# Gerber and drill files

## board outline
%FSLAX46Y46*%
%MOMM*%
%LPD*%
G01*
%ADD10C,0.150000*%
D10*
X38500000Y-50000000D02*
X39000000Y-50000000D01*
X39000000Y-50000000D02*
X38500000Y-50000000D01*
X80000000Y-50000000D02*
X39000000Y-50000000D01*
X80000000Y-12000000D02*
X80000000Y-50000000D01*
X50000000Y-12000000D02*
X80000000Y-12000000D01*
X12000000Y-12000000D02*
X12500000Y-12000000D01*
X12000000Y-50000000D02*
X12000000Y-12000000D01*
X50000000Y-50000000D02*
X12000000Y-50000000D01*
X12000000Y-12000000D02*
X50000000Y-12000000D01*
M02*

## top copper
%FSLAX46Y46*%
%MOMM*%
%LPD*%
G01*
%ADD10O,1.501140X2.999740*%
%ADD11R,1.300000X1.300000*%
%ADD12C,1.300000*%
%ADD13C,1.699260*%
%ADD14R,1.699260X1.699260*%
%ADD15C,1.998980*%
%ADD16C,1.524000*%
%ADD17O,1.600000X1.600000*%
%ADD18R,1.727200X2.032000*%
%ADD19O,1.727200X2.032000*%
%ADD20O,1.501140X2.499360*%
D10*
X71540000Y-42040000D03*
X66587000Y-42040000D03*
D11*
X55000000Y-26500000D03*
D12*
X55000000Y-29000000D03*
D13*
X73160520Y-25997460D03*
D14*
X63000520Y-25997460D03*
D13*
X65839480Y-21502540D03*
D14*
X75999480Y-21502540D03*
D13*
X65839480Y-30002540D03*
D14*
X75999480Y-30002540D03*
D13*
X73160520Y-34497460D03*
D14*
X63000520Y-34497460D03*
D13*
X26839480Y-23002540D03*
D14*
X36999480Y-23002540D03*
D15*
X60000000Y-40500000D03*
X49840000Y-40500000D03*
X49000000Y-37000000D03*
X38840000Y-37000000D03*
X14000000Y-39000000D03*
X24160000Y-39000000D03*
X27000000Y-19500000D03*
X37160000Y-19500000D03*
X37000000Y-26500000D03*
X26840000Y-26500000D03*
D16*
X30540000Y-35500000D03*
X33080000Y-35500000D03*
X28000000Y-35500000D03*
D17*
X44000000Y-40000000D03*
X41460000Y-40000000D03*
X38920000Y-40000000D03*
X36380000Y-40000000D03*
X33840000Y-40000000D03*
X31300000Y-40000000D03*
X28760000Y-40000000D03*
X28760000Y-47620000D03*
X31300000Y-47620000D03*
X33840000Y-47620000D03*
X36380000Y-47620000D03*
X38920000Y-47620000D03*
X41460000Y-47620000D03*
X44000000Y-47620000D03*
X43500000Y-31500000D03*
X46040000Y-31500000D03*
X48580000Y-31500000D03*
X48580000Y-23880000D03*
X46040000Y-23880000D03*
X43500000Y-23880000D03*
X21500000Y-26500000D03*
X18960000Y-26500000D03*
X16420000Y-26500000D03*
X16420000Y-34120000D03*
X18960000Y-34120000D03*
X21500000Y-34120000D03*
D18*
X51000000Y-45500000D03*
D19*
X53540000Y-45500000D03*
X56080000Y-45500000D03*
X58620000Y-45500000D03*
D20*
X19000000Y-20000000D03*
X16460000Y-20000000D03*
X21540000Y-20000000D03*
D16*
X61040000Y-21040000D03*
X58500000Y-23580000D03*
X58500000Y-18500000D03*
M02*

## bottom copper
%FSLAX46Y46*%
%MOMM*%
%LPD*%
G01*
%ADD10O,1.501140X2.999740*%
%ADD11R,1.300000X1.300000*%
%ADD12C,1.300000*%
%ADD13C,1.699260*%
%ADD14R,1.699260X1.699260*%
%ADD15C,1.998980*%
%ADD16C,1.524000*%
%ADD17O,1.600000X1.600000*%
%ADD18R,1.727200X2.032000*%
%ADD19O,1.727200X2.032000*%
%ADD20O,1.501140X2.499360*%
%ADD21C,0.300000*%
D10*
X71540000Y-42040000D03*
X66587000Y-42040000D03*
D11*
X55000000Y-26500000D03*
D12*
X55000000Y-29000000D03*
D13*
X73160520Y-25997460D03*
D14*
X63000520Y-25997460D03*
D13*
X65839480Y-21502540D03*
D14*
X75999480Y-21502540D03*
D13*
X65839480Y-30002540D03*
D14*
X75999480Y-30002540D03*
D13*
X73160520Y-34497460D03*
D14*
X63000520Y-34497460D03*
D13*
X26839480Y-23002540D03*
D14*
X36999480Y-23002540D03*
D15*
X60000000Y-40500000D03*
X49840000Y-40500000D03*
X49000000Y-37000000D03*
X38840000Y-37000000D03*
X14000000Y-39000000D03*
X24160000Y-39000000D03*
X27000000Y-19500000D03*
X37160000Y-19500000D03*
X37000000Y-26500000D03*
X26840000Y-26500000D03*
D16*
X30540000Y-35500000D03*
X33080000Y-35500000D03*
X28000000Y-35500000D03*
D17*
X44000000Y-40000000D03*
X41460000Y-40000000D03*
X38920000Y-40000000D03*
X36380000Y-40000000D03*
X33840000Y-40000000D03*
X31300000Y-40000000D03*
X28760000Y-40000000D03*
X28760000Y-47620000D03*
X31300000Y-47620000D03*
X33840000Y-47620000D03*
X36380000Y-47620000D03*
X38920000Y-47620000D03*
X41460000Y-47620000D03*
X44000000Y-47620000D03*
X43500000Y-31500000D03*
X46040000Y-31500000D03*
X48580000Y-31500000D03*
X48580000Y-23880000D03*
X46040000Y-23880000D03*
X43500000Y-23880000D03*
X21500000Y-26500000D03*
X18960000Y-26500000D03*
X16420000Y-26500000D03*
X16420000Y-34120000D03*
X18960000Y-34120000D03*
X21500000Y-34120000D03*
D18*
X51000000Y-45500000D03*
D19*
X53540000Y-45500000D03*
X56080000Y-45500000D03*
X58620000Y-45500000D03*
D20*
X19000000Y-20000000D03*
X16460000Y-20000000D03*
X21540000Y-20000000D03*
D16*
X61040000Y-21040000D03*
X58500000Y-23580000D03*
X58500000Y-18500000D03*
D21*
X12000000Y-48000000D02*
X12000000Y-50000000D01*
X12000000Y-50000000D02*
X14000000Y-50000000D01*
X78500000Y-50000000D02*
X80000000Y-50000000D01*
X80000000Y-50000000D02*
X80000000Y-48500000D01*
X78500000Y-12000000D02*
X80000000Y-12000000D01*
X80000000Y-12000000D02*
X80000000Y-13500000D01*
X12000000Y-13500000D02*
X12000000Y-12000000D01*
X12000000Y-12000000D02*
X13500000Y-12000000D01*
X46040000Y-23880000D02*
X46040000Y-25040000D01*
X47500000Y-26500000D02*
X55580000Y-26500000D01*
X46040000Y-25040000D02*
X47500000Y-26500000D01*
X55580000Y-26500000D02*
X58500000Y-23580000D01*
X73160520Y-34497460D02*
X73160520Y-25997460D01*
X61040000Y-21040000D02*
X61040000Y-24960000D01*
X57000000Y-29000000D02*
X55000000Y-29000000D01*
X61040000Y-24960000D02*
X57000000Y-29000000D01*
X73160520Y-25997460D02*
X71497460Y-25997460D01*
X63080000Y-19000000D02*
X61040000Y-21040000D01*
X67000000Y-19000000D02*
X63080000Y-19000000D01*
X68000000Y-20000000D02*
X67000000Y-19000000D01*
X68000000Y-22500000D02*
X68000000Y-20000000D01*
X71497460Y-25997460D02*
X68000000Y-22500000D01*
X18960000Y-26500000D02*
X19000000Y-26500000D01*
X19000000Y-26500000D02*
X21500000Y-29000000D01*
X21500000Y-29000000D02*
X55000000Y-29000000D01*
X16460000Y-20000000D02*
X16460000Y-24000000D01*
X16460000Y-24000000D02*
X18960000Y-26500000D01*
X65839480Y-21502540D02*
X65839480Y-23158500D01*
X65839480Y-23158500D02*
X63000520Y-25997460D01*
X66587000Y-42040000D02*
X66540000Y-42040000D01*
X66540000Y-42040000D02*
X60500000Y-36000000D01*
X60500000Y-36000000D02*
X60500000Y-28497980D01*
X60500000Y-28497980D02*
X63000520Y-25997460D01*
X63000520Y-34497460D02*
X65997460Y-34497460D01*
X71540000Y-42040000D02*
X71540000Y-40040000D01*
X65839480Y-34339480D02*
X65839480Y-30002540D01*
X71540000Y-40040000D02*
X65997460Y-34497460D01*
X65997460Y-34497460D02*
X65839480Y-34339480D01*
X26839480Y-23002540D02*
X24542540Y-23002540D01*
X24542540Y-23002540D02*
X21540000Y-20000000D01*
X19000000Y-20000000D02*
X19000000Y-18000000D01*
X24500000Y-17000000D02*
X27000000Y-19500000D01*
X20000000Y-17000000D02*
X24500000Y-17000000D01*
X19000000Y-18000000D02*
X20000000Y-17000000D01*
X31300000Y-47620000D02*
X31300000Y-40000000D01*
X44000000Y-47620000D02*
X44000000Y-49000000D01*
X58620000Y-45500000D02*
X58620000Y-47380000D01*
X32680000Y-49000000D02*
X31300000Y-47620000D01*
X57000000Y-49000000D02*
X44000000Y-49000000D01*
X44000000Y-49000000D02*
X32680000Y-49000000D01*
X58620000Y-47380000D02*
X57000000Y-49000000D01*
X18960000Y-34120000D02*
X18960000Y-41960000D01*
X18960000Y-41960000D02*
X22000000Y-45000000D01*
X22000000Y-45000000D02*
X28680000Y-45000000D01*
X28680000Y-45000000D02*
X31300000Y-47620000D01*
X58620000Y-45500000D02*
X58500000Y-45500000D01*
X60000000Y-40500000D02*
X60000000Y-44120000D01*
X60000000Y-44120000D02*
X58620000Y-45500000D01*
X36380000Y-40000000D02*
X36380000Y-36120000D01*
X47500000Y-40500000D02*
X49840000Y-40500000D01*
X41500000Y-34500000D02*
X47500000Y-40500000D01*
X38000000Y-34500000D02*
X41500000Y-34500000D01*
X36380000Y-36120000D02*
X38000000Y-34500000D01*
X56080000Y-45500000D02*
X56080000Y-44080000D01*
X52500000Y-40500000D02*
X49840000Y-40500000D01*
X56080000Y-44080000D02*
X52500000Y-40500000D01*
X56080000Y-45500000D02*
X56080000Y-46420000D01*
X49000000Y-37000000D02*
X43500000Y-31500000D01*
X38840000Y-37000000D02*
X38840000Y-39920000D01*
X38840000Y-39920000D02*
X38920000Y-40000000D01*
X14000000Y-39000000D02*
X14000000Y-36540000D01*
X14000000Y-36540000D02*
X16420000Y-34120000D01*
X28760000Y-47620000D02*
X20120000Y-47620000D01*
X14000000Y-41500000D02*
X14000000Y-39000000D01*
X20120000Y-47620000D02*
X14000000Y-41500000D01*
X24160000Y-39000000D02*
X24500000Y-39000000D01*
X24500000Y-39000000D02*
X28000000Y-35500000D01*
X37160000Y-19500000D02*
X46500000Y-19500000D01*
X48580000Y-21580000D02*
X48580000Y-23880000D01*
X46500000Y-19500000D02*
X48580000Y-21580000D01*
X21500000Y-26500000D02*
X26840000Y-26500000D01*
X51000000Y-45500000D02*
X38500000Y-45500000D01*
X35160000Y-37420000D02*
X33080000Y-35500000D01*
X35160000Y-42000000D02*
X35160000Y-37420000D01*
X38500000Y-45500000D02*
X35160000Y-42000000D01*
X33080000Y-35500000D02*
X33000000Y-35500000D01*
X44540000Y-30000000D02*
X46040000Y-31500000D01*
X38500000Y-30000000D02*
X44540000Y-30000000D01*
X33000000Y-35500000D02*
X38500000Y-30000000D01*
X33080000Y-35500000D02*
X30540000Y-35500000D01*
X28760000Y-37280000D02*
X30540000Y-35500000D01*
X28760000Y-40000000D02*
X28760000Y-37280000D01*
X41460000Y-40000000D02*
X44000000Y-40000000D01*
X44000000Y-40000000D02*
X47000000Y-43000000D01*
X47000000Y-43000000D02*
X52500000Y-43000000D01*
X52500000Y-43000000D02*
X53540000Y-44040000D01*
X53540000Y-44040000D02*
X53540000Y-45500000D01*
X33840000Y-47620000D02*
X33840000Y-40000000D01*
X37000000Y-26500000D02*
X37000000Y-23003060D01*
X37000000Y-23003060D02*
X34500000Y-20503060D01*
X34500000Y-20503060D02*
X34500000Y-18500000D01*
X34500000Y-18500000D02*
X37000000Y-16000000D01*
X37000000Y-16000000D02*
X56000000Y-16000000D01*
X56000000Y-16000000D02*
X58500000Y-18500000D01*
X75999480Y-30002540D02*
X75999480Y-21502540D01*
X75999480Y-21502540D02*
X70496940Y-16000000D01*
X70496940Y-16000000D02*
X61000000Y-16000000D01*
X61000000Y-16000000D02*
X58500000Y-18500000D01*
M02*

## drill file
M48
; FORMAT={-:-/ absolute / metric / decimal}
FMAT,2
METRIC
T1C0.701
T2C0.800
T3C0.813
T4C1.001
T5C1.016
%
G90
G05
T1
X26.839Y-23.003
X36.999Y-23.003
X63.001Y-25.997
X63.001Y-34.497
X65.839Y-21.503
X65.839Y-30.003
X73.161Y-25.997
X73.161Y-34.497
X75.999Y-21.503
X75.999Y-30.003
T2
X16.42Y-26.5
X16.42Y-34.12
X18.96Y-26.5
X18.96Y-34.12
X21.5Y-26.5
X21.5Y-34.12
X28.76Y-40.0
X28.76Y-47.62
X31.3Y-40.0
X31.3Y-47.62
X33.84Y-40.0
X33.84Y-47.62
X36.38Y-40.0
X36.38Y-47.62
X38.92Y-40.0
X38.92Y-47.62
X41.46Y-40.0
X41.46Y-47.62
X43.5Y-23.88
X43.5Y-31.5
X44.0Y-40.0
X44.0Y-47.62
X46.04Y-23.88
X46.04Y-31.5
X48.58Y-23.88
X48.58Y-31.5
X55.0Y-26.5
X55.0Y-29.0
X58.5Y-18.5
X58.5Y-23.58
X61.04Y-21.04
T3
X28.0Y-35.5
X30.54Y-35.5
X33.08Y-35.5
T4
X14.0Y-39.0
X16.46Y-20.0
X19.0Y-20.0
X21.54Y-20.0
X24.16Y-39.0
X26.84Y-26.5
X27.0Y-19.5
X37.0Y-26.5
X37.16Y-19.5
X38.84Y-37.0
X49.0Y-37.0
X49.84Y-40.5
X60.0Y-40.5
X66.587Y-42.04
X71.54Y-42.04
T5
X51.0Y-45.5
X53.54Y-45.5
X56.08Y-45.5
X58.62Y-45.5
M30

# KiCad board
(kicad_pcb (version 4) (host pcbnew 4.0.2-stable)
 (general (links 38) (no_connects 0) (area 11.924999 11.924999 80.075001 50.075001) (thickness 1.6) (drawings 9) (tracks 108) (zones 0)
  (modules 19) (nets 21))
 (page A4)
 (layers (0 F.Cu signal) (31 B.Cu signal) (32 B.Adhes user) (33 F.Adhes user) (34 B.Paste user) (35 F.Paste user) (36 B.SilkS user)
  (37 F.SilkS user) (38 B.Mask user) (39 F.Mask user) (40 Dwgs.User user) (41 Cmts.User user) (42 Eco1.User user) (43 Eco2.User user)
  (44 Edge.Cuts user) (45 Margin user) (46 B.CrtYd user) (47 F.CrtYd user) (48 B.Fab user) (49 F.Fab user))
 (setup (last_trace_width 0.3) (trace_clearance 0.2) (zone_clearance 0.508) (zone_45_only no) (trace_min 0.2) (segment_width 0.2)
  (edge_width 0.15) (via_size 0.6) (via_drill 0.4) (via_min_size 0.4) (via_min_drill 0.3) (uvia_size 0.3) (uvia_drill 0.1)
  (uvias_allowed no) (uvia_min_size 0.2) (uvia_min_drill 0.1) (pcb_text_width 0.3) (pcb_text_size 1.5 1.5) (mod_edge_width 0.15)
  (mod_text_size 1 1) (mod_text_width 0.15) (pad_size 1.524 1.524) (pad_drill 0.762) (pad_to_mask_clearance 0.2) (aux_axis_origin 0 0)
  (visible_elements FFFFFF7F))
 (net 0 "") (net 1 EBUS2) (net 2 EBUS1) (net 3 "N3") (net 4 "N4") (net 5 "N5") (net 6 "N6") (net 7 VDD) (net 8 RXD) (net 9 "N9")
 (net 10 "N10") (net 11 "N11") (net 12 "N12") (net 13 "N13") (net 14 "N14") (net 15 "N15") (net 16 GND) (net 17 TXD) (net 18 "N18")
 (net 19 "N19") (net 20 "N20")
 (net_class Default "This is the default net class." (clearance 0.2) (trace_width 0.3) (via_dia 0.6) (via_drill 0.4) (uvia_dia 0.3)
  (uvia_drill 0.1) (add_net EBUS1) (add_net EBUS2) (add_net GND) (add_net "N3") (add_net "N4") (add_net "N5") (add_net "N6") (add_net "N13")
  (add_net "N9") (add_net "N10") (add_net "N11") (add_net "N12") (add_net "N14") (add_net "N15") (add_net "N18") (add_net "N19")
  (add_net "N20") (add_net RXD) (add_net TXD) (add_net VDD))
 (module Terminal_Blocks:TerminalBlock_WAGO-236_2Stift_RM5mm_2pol (layer F.Cu) (at 69 39.5 180)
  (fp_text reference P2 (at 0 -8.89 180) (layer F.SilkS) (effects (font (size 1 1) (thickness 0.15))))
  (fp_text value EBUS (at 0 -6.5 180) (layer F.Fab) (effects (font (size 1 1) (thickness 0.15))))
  (pad 1 thru_hole oval (at -2.54 -2.54 270) (size 2.99974 1.50114) (drill 1.00076) (layers *.Cu *.Mask F.SilkS) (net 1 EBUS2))
  (pad 2 thru_hole oval (at 2.413 -2.54 270) (size 2.99974 1.50114) (drill 1.00076) (layers *.Cu *.Mask F.SilkS) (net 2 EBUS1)))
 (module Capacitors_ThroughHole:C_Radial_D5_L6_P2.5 (layer F.Cu) (at 55 26.5 270)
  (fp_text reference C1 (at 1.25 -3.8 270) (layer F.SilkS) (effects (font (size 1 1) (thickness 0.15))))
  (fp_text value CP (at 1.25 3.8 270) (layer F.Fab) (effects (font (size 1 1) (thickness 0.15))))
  (pad 1 thru_hole rect (at 0 0 270) (size 1.3 1.3) (drill 0.8) (layers *.Cu *.Mask F.SilkS) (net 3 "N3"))
  (pad 2 thru_hole circle (at 2.5 0 270) (size 1.3 1.3) (drill 0.8) (layers *.Cu *.Mask F.SilkS) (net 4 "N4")))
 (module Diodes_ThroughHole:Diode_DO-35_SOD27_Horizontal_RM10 (layer F.Cu) (at 63 26)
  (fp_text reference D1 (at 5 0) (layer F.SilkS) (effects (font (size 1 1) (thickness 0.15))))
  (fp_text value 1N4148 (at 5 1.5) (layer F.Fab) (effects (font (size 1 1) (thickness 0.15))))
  (pad 2 thru_hole circle (at 10.16052 -0.00254 180) (size 1.69926 1.69926) (drill 0.70104) (layers *.Cu *.Mask F.SilkS) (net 4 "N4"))
  (pad 1 thru_hole rect (at 0.00052 -0.00254 180) (size 1.69926 1.69926) (drill 0.70104) (layers *.Cu *.Mask F.SilkS) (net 2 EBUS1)))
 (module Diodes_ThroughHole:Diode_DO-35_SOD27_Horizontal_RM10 (layer F.Cu) (at 76 21.5 180)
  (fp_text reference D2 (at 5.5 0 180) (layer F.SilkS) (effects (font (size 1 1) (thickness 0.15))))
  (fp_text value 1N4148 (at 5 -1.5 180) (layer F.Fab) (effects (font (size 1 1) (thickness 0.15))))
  (pad 2 thru_hole circle (at 10.16052 -0.00254) (size 1.69926 1.69926) (drill 0.70104) (layers *.Cu *.Mask F.SilkS) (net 2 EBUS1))
  (pad 1 thru_hole rect (at 0.00052 -0.00254) (size 1.69926 1.69926) (drill 0.70104) (layers *.Cu *.Mask F.SilkS) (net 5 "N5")))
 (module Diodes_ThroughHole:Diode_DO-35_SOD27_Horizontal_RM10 (layer F.Cu) (at 76 30 180)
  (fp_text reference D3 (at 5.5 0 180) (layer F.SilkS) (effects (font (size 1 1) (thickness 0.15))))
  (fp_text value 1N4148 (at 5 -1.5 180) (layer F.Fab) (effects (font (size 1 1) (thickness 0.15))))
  (pad 2 thru_hole circle (at 10.16052 -0.00254) (size 1.69926 1.69926) (drill 0.70104) (layers *.Cu *.Mask F.SilkS) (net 1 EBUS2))
  (pad 1 thru_hole rect (at 0.00052 -0.00254) (size 1.69926 1.69926) (drill 0.70104) (layers *.Cu *.Mask F.SilkS) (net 5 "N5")))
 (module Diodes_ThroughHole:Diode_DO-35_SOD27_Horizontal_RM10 (layer F.Cu) (at 63 34.5)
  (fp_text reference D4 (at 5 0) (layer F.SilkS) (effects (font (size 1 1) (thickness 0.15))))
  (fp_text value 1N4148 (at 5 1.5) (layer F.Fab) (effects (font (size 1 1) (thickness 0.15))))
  (pad 2 thru_hole circle (at 10.16052 -0.00254 180) (size 1.69926 1.69926) (drill 0.70104) (layers *.Cu *.Mask F.SilkS) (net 4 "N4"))
  (pad 1 thru_hole rect (at 0.00052 -0.00254 180) (size 1.69926 1.69926) (drill 0.70104) (layers *.Cu *.Mask F.SilkS) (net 1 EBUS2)))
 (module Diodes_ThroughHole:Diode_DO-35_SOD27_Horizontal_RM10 (layer F.Cu) (at 37 23 180)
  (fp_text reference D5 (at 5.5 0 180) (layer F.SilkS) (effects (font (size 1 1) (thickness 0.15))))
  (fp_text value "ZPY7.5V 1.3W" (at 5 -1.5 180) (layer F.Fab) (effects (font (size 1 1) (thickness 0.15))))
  (pad 2 thru_hole circle (at 10.16052 -0.00254) (size 1.69926 1.69926) (drill 0.70104) (layers *.Cu *.Mask F.SilkS) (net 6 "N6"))
  (pad 1 thru_hole rect (at 0.00052 -0.00254) (size 1.69926 1.69926) (drill 0.70104) (layers *.Cu *.Mask F.SilkS) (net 5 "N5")))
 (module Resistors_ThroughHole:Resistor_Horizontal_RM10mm (layer F.Cu) (at 60 40.5 180)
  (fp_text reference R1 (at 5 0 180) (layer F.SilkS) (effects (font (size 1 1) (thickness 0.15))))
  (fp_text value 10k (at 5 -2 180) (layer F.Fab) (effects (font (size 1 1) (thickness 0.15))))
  (pad 1 thru_hole circle (at 0 0 180) (size 1.99898 1.99898) (drill 1.00076) (layers *.Cu *.SilkS *.Mask) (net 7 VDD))
  (pad 2 thru_hole circle (at 10.16 0 180) (size 1.99898 1.99898) (drill 1.00076) (layers *.Cu *.SilkS *.Mask) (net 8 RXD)))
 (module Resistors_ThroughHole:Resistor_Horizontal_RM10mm (layer F.Cu) (at 49 37 180)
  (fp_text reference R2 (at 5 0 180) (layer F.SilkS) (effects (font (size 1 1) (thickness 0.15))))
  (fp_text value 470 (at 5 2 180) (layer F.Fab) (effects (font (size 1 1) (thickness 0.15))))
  (pad 1 thru_hole circle (at 0 0 180) (size 1.99898 1.99898) (drill 1.00076) (layers *.Cu *.SilkS *.Mask) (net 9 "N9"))
  (pad 2 thru_hole circle (at 10.16 0 180) (size 1.99898 1.99898) (drill 1.00076) (layers *.Cu *.SilkS *.Mask) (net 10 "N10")))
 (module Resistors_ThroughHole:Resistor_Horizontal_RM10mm (layer F.Cu) (at 14 39)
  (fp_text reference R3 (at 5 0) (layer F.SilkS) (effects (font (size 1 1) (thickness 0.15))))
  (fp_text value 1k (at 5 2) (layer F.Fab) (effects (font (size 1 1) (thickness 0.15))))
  (pad 1 thru_hole circle (at 0 0) (size 1.99898 1.99898) (drill 1.00076) (layers *.Cu *.SilkS *.Mask) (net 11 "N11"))
  (pad 2 thru_hole circle (at 10.16 0) (size 1.99898 1.99898) (drill 1.00076) (layers *.Cu *.SilkS *.Mask) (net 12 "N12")))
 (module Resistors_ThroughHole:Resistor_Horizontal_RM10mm (layer F.Cu) (at 27 19.5)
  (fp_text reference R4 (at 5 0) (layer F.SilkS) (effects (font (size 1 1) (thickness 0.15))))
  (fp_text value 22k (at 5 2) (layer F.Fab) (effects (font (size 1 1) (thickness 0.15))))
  (pad 1 thru_hole circle (at 0 0) (size 1.99898 1.99898) (drill 1.00076) (layers *.Cu *.SilkS *.Mask) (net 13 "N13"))
  (pad 2 thru_hole circle (at 10.16 0) (size 1.99898 1.99898) (drill 1.00076) (layers *.Cu *.SilkS *.Mask) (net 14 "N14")))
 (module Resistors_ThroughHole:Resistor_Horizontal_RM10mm (layer F.Cu) (at 37 26.5 180)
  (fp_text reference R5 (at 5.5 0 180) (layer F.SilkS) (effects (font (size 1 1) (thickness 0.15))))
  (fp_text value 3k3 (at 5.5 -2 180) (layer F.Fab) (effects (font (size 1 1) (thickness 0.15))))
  (pad 1 thru_hole circle (at 0 0 180) (size 1.99898 1.99898) (drill 1.00076) (layers *.Cu *.SilkS *.Mask) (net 5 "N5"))
  (pad 2 thru_hole circle (at 10.16 0 180) (size 1.99898 1.99898) (drill 1.00076) (layers *.Cu *.SilkS *.Mask) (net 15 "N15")))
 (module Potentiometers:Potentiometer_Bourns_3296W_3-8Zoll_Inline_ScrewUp (layer F.Cu) (at 28 35.5 270)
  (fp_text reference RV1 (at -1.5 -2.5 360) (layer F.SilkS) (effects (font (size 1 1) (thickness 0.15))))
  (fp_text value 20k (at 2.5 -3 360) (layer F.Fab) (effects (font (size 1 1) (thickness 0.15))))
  (pad 2 thru_hole circle (at 0 -2.54 270) (size 1.524 1.524) (drill 0.8128) (layers *.Cu *.Mask F.SilkS) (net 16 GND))
  (pad 3 thru_hole circle (at 0 -5.08 270) (size 1.524 1.524) (drill 0.8128) (layers *.Cu *.Mask F.SilkS) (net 16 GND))
  (pad 1 thru_hole circle (at 0 0 270) (size 1.524 1.524) (drill 0.8128) (layers *.Cu *.Mask F.SilkS) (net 12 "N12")))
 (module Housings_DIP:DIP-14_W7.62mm (layer F.Cu) (at 44 40 270)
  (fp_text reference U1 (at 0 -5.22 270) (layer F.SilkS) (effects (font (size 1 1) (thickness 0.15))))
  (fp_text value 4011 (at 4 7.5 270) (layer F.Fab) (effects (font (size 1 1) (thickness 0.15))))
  (pad 1 thru_hole oval (at 0 0 270) (size 1.6 1.6) (drill 0.8) (layers *.Cu *.Mask F.SilkS) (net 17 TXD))
  (pad 2 thru_hole oval (at 0 2.54 270) (size 1.6 1.6) (drill 0.8) (layers *.Cu *.Mask F.SilkS) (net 17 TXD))
  (pad 3 thru_hole oval (at 0 5.08 270) (size 1.6 1.6) (drill 0.8) (layers *.Cu *.Mask F.SilkS) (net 10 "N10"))
  (pad 4 thru_hole oval (at 0 7.62 270) (size 1.6 1.6) (drill 0.8) (layers *.Cu *.Mask F.SilkS) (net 8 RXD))
  (pad 5 thru_hole oval (at 0 10.16 270) (size 1.6 1.6) (drill 0.8) (layers *.Cu *.Mask F.SilkS) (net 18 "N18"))
  (pad 6 thru_hole oval (at 0 12.7 270) (size 1.6 1.6) (drill 0.8) (layers *.Cu *.Mask F.SilkS) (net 7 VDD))
  (pad 7 thru_hole oval (at 0 15.24 270) (size 1.6 1.6) (drill 0.8) (layers *.Cu *.Mask F.SilkS) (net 16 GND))
  (pad 8 thru_hole oval (at 7.62 15.24 270) (size 1.6 1.6) (drill 0.8) (layers *.Cu *.Mask F.SilkS) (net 11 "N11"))
  (pad 9 thru_hole oval (at 7.62 12.7 270) (size 1.6 1.6) (drill 0.8) (layers *.Cu *.Mask F.SilkS) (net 7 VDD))
  (pad 10 thru_hole oval (at 7.62 10.16 270) (size 1.6 1.6) (drill 0.8) (layers *.Cu *.Mask F.SilkS) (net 18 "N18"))
  (pad 11 thru_hole oval (at 7.62 7.62 270) (size 1.6 1.6) (drill 0.8) (layers *.Cu *.Mask F.SilkS))
  (pad 12 thru_hole oval (at 7.62 5.08 270) (size 1.6 1.6) (drill 0.8) (layers *.Cu *.Mask F.SilkS))
  (pad 13 thru_hole oval (at 7.62 2.54 270) (size 1.6 1.6) (drill 0.8) (layers *.Cu *.Mask F.SilkS))
  (pad 14 thru_hole oval (at 7.62 0 270) (size 1.6 1.6) (drill 0.8) (layers *.Cu *.Mask F.SilkS) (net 7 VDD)))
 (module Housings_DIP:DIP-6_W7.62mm (layer F.Cu) (at 43.5 31.5 90)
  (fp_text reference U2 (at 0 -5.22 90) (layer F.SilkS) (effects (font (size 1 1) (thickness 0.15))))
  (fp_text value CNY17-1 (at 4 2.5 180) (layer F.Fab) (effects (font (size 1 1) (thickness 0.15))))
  (pad 1 thru_hole oval (at 0 0 90) (size 1.6 1.6) (drill 0.8) (layers *.Cu *.Mask F.SilkS) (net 9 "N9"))
  (pad 2 thru_hole oval (at 0 2.54 90) (size 1.6 1.6) (drill 0.8) (layers *.Cu *.Mask F.SilkS) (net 16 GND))
  (pad 3 thru_hole oval (at 0 5.08 90) (size 1.6 1.6) (drill 0.8) (layers *.Cu *.Mask F.SilkS))
  (pad 4 thru_hole oval (at 7.62 5.08 90) (size 1.6 1.6) (drill 0.8) (layers *.Cu *.Mask F.SilkS) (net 14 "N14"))
  (pad 5 thru_hole oval (at 7.62 2.54 90) (size 1.6 1.6) (drill 0.8) (layers *.Cu *.Mask F.SilkS) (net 3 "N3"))
  (pad 6 thru_hole oval (at 7.62 0 90) (size 1.6 1.6) (drill 0.8) (layers *.Cu *.Mask F.SilkS) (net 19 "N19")))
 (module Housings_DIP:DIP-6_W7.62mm (layer F.Cu) (at 21.5 26.5 270)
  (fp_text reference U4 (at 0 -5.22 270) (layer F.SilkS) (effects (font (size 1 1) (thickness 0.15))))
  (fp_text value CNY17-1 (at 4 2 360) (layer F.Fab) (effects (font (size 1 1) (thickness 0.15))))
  (pad 1 thru_hole oval (at 0 0 270) (size 1.6 1.6) (drill 0.8) (layers *.Cu *.Mask F.SilkS) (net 15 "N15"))
  (pad 2 thru_hole oval (at 0 2.54 270) (size 1.6 1.6) (drill 0.8) (layers *.Cu *.Mask F.SilkS) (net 4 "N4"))
  (pad 3 thru_hole oval (at 0 5.08 270) (size 1.6 1.6) (drill 0.8) (layers *.Cu *.Mask F.SilkS))
  (pad 4 thru_hole oval (at 7.62 5.08 270) (size 1.6 1.6) (drill 0.8) (layers *.Cu *.Mask F.SilkS) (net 11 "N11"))
  (pad 5 thru_hole oval (at 7.62 2.54 270) (size 1.6 1.6) (drill 0.8) (layers *.Cu *.Mask F.SilkS) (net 7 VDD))
  (pad 6 thru_hole oval (at 7.62 0 270) (size 1.6 1.6) (drill 0.8) (layers *.Cu *.Mask F.SilkS) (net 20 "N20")))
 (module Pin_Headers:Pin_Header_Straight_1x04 (layer F.Cu) (at 51 45.5 90)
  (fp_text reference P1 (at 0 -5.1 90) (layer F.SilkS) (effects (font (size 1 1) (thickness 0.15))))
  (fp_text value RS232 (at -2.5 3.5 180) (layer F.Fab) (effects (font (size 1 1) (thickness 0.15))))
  (pad 1 thru_hole rect (at 0 0 90) (size 2.032 1.7272) (drill 1.016) (layers *.Cu *.Mask F.SilkS) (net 16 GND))
  (pad 2 thru_hole oval (at 0 2.54 90) (size 2.032 1.7272) (drill 1.016) (layers *.Cu *.Mask F.SilkS) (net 17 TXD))
  (pad 3 thru_hole oval (at 0 5.08 90) (size 2.032 1.7272) (drill 1.016) (layers *.Cu *.Mask F.SilkS) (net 8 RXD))
  (pad 4 thru_hole oval (at 0 7.62 90) (size 2.032 1.7272) (drill 1.016) (layers *.Cu *.Mask F.SilkS) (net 7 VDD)))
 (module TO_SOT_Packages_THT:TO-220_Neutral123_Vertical (layer F.Cu) (at 19 20)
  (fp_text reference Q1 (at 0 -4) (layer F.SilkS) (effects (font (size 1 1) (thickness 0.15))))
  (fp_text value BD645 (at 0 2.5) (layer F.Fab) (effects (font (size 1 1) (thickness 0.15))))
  (pad 2 thru_hole oval (at 0 0 90) (size 2.49936 1.50114) (drill 1.00076) (layers *.Cu *.Mask F.SilkS) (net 13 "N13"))
  (pad 1 thru_hole oval (at -2.54 0 90) (size 2.49936 1.50114) (drill 1.00076) (layers *.Cu *.Mask F.SilkS) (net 4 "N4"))
  (pad 3 thru_hole oval (at 2.54 0 90) (size 2.49936 1.50114) (drill 1.00076) (layers *.Cu *.Mask F.SilkS) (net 6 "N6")))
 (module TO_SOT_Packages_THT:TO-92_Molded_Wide (layer F.Cu) (at 58.5 18.5 270)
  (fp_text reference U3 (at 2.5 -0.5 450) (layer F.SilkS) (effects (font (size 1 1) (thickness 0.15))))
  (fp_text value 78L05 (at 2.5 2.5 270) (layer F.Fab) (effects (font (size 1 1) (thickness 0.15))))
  (pad 2 thru_hole circle (at 2.54 -2.54) (size 1.524 1.524) (drill 0.8) (layers *.Cu *.Mask F.SilkS) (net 4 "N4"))
  (pad 3 thru_hole circle (at 5.08 0) (size 1.524 1.524) (drill 0.8) (layers *.Cu *.Mask F.SilkS) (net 3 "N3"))
  (pad 1 thru_hole circle (at 0 0) (size 1.524 1.524) (drill 0.8) (layers *.Cu *.Mask F.SilkS) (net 5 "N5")))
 (gr_line (start 38.5 50) (end 39 50) (angle 90) (layer Edge.Cuts) (width 0.15))
 (gr_line (start 39 50) (end 38.5 50) (angle 90) (layer Edge.Cuts) (width 0.15))
 (gr_line (start 80 50) (end 39 50) (angle 90) (layer Edge.Cuts) (width 0.15))
 (gr_line (start 80 12) (end 80 50) (angle 90) (layer Edge.Cuts) (width 0.15))
 (gr_line (start 50 12) (end 80 12) (angle 90) (layer Edge.Cuts) (width 0.15))
 (gr_line (start 12 12) (end 12.5 12) (angle 90) (layer Edge.Cuts) (width 0.15))
 (gr_line (start 12 50) (end 12 12) (angle 90) (layer Edge.Cuts) (width 0.15))
 (gr_line (start 50 50) (end 12 50) (angle 90) (layer Edge.Cuts) (width 0.15))
 (gr_line (start 12 12) (end 50 12) (angle 90) (layer Edge.Cuts) (width 0.15))
 (segment (start 12 48) (end 12 50) (width 0.3) (layer B.Cu) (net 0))
 (segment (start 12 50) (end 14 50) (width 0.3) (layer B.Cu) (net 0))
 (segment (start 78.5 50) (end 80 50) (width 0.3) (layer B.Cu) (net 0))
 (segment (start 80 50) (end 80 48.5) (width 0.3) (layer B.Cu) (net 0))
 (segment (start 78.5 12) (end 80 12) (width 0.3) (layer B.Cu) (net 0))
 (segment (start 80 12) (end 80 13.5) (width 0.3) (layer B.Cu) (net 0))
 (segment (start 12 13.5) (end 12 12) (width 0.3) (layer B.Cu) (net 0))
 (segment (start 12 12) (end 13.5 12) (width 0.3) (layer B.Cu) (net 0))
 (segment (start 46.04 23.88) (end 46.04 25.04) (width 0.3) (layer B.Cu) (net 3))
 (segment (start 47.5 26.5) (end 55.58 26.5) (width 0.3) (layer B.Cu) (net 3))
 (segment (start 46.04 25.04) (end 47.5 26.5) (width 0.3) (layer B.Cu) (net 3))
 (segment (start 55.58 26.5) (end 58.5 23.58) (width 0.3) (layer B.Cu) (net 3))
 (segment (start 73.16052 34.49746) (end 73.16052 25.99746) (width 0.3) (layer B.Cu) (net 4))
 (segment (start 61.04 21.04) (end 61.04 24.96) (width 0.3) (layer B.Cu) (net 4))
 (segment (start 57 29) (end 55 29) (width 0.3) (layer B.Cu) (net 4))
 (segment (start 61.04 24.96) (end 57 29) (width 0.3) (layer B.Cu) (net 4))
 (segment (start 73.16052 25.99746) (end 71.49746 25.99746) (width 0.3) (layer B.Cu) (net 4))
 (segment (start 63.08 19) (end 61.04 21.04) (width 0.3) (layer B.Cu) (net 4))
 (segment (start 67 19) (end 63.08 19) (width 0.3) (layer B.Cu) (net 4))
 (segment (start 68 20) (end 67 19) (width 0.3) (layer B.Cu) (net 4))
 (segment (start 68 22.5) (end 68 20) (width 0.3) (layer B.Cu) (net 4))
 (segment (start 71.49746 25.99746) (end 68 22.5) (width 0.3) (layer B.Cu) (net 4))
 (segment (start 18.96 26.5) (end 19 26.5) (width 0.3) (layer B.Cu) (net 4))
 (segment (start 19 26.5) (end 21.5 29) (width 0.3) (layer B.Cu) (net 4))
 (segment (start 21.5 29) (end 55 29) (width 0.3) (layer B.Cu) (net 4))
 (segment (start 16.46 20) (end 16.46 24) (width 0.3) (layer B.Cu) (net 4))
 (segment (start 16.46 24) (end 18.96 26.5) (width 0.3) (layer B.Cu) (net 4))
 (segment (start 65.83948 21.50254) (end 65.83948 23.1585) (width 0.3) (layer B.Cu) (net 2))
 (segment (start 65.83948 23.1585) (end 63.00052 25.99746) (width 0.3) (layer B.Cu) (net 2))
 (segment (start 66.587 42.04) (end 66.54 42.04) (width 0.3) (layer B.Cu) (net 2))
 (segment (start 66.54 42.04) (end 60.5 36) (width 0.3) (layer B.Cu) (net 2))
 (segment (start 60.5 36) (end 60.5 28.49798) (width 0.3) (layer B.Cu) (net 2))
 (segment (start 60.5 28.49798) (end 63.00052 25.99746) (width 0.3) (layer B.Cu) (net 2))
 (segment (start 63.00052 34.49746) (end 65.99746 34.49746) (width 0.3) (layer B.Cu) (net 1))
 (segment (start 71.54 42.04) (end 71.54 40.04) (width 0.3) (layer B.Cu) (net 1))
 (segment (start 65.83948 34.33948) (end 65.83948 30.00254) (width 0.3) (layer B.Cu) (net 1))
 (segment (start 71.54 40.04) (end 65.99746 34.49746) (width 0.3) (layer B.Cu) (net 1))
 (segment (start 65.99746 34.49746) (end 65.83948 34.33948) (width 0.3) (layer B.Cu) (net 1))
 (segment (start 26.83948 23.00254) (end 24.54254 23.00254) (width 0.3) (layer B.Cu) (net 6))
 (segment (start 24.54254 23.00254) (end 21.54 20) (width 0.3) (layer B.Cu) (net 6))
 (segment (start 19 20) (end 19 18) (width 0.3) (layer B.Cu) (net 13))
 (segment (start 24.5 17) (end 27 19.5) (width 0.3) (layer B.Cu) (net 13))
 (segment (start 20 17) (end 24.5 17) (width 0.3) (layer B.Cu) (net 13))
 (segment (start 19 18) (end 20 17) (width 0.3) (layer B.Cu) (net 13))
 (segment (start 31.3 47.62) (end 31.3 40) (width 0.3) (layer B.Cu) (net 7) (status C00000))
 (segment (start 44 47.62) (end 44 49) (width 0.3) (layer B.Cu) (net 7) (status 400000))
 (segment (start 58.62 45.5) (end 58.62 47.38) (width 0.3) (layer B.Cu) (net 7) (status 400000))
 (segment (start 32.68 49) (end 31.3 47.62) (width 0.3) (layer B.Cu) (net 7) (status 800000))
 (segment (start 57 49) (end 44 49) (width 0.3) (layer B.Cu) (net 7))
 (segment (start 44 49) (end 32.68 49) (width 0.3) (layer B.Cu) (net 7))
 (segment (start 58.62 47.38) (end 57 49) (width 0.3) (layer B.Cu) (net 7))
 (segment (start 18.96 34.12) (end 18.96 41.96) (width 0.3) (layer B.Cu) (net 7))
 (segment (start 18.96 41.96) (end 22 45) (width 0.3) (layer B.Cu) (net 7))
 (segment (start 22 45) (end 28.68 45) (width 0.3) (layer B.Cu) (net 7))
 (segment (start 28.68 45) (end 31.3 47.62) (width 0.3) (layer B.Cu) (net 7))
 (segment (start 58.62 45.5) (end 58.5 45.5) (width 0.3) (layer B.Cu) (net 7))
 (segment (start 60 40.5) (end 60 44.12) (width 0.3) (layer B.Cu) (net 7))
 (segment (start 60 44.12) (end 58.62 45.5) (width 0.3) (layer B.Cu) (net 7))
 (segment (start 36.38 40) (end 36.38 36.12) (width 0.3) (layer B.Cu) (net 8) (status 400000))
 (segment (start 47.5 40.5) (end 49.84 40.5) (width 0.3) (layer B.Cu) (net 8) (status 800000))
 (segment (start 41.5 34.5) (end 47.5 40.5) (width 0.3) (layer B.Cu) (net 8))
 (segment (start 38 34.5) (end 41.5 34.5) (width 0.3) (layer B.Cu) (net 8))
 (segment (start 36.38 36.12) (end 38 34.5) (width 0.3) (layer B.Cu) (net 8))
 (segment (start 56.08 45.5) (end 56.08 44.08) (width 0.3) (layer B.Cu) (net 8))
 (segment (start 52.5 40.5) (end 49.84 40.5) (width 0.3) (layer B.Cu) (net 8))
 (segment (start 56.08 44.08) (end 52.5 40.5) (width 0.3) (layer B.Cu) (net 8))
 (segment (start 56.08 45.5) (end 56.08 46.42) (width 0.3) (layer B.Cu) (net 8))
 (segment (start 49 37) (end 43.5 31.5) (width 0.3) (layer B.Cu) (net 9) (status C00000))
 (segment (start 38.84 37) (end 38.84 39.92) (width 0.3) (layer B.Cu) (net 10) (status C00000))
 (segment (start 38.84 39.92) (end 38.92 40) (width 0.3) (layer B.Cu) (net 10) (status C00000))
 (segment (start 14 39) (end 14 36.54) (width 0.3) (layer B.Cu) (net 11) (status 400000))
 (segment (start 14 36.54) (end 16.42 34.12) (width 0.3) (layer B.Cu) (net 11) (status 800000))
 (segment (start 28.76 47.62) (end 20.12 47.62) (width 0.3) (layer B.Cu) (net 11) (status 400000))
 (segment (start 14 41.5) (end 14 39) (width 0.3) (layer B.Cu) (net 11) (status 800000))
 (segment (start 20.12 47.62) (end 14 41.5) (width 0.3) (layer B.Cu) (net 11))
 (segment (start 24.16 39) (end 24.5 39) (width 0.3) (layer B.Cu) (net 12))
 (segment (start 24.5 39) (end 28 35.5) (width 0.3) (layer B.Cu) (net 12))
 (segment (start 37.16 19.5) (end 46.5 19.5) (width 0.3) (layer B.Cu) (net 14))
 (segment (start 48.58 21.58) (end 48.58 23.88) (width 0.3) (layer B.Cu) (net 14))
 (segment (start 46.5 19.5) (end 48.58 21.58) (width 0.3) (layer B.Cu) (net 14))
 (segment (start 21.5 26.5) (end 26.84 26.5) (width 0.3) (layer B.Cu) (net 15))
 (segment (start 51 45.5) (end 38.5 45.5) (width 0.3) (layer B.Cu) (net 16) (status 400000))
 (segment (start 35.16 37.42) (end 33.08 35.5) (width 0.3) (layer B.Cu) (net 16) (status 800000))
 (segment (start 35.16 42) (end 35.16 37.42) (width 0.3) (layer B.Cu) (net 16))
 (segment (start 38.5 45.5) (end 35.16 42) (width 0.3) (layer B.Cu) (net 16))
 (segment (start 33.08 35.5) (end 33 35.5) (width 0.3) (layer B.Cu) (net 16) (status 400000))
 (segment (start 44.54 30) (end 46.04 31.5) (width 0.3) (layer B.Cu) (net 16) (status 800000))
 (segment (start 38.5 30) (end 44.54 30) (width 0.3) (layer B.Cu) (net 16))
 (segment (start 33 35.5) (end 38.5 30) (width 0.3) (layer B.Cu) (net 16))
 (segment (start 33.08 35.5) (end 30.54 35.5) (width 0.3) (layer B.Cu) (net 16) (status C00000))
 (segment (start 28.76 37.28) (end 30.54 35.5) (width 0.3) (layer B.Cu) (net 16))
 (segment (start 28.76 40) (end 28.76 37.28) (width 0.3) (layer B.Cu) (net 16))
 (segment (start 41.46 40) (end 44 40) (width 0.3) (layer B.Cu) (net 17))
 (segment (start 44 40) (end 47 43) (width 0.3) (layer B.Cu) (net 17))
 (segment (start 47 43) (end 52.5 43) (width 0.3) (layer B.Cu) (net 17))
 (segment (start 52.5 43) (end 53.54 44.04) (width 0.3) (layer B.Cu) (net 17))
 (segment (start 53.54 44.04) (end 53.54 45.5) (width 0.3) (layer B.Cu) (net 17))
 (segment (start 33.84 47.62) (end 33.84 40) (width 0.3) (layer B.Cu) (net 18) (status C00000))
 (segment (start 37 26.5) (end 37 23.00306) (width 0.3) (layer B.Cu) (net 5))
 (segment (start 37 23.00306) (end 34.5 20.50306) (width 0.3) (layer B.Cu) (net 5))
 (segment (start 34.5 20.50306) (end 34.5 18.5) (width 0.3) (layer B.Cu) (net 5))
 (segment (start 34.5 18.5) (end 37 16) (width 0.3) (layer B.Cu) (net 5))
 (segment (start 37 16) (end 56 16) (width 0.3) (layer B.Cu) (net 5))
 (segment (start 56 16) (end 58.5 18.5) (width 0.3) (layer B.Cu) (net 5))
 (segment (start 75.99948 30.00254) (end 75.99948 21.50254) (width 0.3) (layer B.Cu) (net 5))
 (segment (start 75.99948 21.50254) (end 70.49694 16) (width 0.3) (layer B.Cu) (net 5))
 (segment (start 70.49694 16) (end 61 16) (width 0.3) (layer B.Cu) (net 5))
 (segment (start 61 16) (end 58.5 18.5) (width 0.3) (layer B.Cu) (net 5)))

